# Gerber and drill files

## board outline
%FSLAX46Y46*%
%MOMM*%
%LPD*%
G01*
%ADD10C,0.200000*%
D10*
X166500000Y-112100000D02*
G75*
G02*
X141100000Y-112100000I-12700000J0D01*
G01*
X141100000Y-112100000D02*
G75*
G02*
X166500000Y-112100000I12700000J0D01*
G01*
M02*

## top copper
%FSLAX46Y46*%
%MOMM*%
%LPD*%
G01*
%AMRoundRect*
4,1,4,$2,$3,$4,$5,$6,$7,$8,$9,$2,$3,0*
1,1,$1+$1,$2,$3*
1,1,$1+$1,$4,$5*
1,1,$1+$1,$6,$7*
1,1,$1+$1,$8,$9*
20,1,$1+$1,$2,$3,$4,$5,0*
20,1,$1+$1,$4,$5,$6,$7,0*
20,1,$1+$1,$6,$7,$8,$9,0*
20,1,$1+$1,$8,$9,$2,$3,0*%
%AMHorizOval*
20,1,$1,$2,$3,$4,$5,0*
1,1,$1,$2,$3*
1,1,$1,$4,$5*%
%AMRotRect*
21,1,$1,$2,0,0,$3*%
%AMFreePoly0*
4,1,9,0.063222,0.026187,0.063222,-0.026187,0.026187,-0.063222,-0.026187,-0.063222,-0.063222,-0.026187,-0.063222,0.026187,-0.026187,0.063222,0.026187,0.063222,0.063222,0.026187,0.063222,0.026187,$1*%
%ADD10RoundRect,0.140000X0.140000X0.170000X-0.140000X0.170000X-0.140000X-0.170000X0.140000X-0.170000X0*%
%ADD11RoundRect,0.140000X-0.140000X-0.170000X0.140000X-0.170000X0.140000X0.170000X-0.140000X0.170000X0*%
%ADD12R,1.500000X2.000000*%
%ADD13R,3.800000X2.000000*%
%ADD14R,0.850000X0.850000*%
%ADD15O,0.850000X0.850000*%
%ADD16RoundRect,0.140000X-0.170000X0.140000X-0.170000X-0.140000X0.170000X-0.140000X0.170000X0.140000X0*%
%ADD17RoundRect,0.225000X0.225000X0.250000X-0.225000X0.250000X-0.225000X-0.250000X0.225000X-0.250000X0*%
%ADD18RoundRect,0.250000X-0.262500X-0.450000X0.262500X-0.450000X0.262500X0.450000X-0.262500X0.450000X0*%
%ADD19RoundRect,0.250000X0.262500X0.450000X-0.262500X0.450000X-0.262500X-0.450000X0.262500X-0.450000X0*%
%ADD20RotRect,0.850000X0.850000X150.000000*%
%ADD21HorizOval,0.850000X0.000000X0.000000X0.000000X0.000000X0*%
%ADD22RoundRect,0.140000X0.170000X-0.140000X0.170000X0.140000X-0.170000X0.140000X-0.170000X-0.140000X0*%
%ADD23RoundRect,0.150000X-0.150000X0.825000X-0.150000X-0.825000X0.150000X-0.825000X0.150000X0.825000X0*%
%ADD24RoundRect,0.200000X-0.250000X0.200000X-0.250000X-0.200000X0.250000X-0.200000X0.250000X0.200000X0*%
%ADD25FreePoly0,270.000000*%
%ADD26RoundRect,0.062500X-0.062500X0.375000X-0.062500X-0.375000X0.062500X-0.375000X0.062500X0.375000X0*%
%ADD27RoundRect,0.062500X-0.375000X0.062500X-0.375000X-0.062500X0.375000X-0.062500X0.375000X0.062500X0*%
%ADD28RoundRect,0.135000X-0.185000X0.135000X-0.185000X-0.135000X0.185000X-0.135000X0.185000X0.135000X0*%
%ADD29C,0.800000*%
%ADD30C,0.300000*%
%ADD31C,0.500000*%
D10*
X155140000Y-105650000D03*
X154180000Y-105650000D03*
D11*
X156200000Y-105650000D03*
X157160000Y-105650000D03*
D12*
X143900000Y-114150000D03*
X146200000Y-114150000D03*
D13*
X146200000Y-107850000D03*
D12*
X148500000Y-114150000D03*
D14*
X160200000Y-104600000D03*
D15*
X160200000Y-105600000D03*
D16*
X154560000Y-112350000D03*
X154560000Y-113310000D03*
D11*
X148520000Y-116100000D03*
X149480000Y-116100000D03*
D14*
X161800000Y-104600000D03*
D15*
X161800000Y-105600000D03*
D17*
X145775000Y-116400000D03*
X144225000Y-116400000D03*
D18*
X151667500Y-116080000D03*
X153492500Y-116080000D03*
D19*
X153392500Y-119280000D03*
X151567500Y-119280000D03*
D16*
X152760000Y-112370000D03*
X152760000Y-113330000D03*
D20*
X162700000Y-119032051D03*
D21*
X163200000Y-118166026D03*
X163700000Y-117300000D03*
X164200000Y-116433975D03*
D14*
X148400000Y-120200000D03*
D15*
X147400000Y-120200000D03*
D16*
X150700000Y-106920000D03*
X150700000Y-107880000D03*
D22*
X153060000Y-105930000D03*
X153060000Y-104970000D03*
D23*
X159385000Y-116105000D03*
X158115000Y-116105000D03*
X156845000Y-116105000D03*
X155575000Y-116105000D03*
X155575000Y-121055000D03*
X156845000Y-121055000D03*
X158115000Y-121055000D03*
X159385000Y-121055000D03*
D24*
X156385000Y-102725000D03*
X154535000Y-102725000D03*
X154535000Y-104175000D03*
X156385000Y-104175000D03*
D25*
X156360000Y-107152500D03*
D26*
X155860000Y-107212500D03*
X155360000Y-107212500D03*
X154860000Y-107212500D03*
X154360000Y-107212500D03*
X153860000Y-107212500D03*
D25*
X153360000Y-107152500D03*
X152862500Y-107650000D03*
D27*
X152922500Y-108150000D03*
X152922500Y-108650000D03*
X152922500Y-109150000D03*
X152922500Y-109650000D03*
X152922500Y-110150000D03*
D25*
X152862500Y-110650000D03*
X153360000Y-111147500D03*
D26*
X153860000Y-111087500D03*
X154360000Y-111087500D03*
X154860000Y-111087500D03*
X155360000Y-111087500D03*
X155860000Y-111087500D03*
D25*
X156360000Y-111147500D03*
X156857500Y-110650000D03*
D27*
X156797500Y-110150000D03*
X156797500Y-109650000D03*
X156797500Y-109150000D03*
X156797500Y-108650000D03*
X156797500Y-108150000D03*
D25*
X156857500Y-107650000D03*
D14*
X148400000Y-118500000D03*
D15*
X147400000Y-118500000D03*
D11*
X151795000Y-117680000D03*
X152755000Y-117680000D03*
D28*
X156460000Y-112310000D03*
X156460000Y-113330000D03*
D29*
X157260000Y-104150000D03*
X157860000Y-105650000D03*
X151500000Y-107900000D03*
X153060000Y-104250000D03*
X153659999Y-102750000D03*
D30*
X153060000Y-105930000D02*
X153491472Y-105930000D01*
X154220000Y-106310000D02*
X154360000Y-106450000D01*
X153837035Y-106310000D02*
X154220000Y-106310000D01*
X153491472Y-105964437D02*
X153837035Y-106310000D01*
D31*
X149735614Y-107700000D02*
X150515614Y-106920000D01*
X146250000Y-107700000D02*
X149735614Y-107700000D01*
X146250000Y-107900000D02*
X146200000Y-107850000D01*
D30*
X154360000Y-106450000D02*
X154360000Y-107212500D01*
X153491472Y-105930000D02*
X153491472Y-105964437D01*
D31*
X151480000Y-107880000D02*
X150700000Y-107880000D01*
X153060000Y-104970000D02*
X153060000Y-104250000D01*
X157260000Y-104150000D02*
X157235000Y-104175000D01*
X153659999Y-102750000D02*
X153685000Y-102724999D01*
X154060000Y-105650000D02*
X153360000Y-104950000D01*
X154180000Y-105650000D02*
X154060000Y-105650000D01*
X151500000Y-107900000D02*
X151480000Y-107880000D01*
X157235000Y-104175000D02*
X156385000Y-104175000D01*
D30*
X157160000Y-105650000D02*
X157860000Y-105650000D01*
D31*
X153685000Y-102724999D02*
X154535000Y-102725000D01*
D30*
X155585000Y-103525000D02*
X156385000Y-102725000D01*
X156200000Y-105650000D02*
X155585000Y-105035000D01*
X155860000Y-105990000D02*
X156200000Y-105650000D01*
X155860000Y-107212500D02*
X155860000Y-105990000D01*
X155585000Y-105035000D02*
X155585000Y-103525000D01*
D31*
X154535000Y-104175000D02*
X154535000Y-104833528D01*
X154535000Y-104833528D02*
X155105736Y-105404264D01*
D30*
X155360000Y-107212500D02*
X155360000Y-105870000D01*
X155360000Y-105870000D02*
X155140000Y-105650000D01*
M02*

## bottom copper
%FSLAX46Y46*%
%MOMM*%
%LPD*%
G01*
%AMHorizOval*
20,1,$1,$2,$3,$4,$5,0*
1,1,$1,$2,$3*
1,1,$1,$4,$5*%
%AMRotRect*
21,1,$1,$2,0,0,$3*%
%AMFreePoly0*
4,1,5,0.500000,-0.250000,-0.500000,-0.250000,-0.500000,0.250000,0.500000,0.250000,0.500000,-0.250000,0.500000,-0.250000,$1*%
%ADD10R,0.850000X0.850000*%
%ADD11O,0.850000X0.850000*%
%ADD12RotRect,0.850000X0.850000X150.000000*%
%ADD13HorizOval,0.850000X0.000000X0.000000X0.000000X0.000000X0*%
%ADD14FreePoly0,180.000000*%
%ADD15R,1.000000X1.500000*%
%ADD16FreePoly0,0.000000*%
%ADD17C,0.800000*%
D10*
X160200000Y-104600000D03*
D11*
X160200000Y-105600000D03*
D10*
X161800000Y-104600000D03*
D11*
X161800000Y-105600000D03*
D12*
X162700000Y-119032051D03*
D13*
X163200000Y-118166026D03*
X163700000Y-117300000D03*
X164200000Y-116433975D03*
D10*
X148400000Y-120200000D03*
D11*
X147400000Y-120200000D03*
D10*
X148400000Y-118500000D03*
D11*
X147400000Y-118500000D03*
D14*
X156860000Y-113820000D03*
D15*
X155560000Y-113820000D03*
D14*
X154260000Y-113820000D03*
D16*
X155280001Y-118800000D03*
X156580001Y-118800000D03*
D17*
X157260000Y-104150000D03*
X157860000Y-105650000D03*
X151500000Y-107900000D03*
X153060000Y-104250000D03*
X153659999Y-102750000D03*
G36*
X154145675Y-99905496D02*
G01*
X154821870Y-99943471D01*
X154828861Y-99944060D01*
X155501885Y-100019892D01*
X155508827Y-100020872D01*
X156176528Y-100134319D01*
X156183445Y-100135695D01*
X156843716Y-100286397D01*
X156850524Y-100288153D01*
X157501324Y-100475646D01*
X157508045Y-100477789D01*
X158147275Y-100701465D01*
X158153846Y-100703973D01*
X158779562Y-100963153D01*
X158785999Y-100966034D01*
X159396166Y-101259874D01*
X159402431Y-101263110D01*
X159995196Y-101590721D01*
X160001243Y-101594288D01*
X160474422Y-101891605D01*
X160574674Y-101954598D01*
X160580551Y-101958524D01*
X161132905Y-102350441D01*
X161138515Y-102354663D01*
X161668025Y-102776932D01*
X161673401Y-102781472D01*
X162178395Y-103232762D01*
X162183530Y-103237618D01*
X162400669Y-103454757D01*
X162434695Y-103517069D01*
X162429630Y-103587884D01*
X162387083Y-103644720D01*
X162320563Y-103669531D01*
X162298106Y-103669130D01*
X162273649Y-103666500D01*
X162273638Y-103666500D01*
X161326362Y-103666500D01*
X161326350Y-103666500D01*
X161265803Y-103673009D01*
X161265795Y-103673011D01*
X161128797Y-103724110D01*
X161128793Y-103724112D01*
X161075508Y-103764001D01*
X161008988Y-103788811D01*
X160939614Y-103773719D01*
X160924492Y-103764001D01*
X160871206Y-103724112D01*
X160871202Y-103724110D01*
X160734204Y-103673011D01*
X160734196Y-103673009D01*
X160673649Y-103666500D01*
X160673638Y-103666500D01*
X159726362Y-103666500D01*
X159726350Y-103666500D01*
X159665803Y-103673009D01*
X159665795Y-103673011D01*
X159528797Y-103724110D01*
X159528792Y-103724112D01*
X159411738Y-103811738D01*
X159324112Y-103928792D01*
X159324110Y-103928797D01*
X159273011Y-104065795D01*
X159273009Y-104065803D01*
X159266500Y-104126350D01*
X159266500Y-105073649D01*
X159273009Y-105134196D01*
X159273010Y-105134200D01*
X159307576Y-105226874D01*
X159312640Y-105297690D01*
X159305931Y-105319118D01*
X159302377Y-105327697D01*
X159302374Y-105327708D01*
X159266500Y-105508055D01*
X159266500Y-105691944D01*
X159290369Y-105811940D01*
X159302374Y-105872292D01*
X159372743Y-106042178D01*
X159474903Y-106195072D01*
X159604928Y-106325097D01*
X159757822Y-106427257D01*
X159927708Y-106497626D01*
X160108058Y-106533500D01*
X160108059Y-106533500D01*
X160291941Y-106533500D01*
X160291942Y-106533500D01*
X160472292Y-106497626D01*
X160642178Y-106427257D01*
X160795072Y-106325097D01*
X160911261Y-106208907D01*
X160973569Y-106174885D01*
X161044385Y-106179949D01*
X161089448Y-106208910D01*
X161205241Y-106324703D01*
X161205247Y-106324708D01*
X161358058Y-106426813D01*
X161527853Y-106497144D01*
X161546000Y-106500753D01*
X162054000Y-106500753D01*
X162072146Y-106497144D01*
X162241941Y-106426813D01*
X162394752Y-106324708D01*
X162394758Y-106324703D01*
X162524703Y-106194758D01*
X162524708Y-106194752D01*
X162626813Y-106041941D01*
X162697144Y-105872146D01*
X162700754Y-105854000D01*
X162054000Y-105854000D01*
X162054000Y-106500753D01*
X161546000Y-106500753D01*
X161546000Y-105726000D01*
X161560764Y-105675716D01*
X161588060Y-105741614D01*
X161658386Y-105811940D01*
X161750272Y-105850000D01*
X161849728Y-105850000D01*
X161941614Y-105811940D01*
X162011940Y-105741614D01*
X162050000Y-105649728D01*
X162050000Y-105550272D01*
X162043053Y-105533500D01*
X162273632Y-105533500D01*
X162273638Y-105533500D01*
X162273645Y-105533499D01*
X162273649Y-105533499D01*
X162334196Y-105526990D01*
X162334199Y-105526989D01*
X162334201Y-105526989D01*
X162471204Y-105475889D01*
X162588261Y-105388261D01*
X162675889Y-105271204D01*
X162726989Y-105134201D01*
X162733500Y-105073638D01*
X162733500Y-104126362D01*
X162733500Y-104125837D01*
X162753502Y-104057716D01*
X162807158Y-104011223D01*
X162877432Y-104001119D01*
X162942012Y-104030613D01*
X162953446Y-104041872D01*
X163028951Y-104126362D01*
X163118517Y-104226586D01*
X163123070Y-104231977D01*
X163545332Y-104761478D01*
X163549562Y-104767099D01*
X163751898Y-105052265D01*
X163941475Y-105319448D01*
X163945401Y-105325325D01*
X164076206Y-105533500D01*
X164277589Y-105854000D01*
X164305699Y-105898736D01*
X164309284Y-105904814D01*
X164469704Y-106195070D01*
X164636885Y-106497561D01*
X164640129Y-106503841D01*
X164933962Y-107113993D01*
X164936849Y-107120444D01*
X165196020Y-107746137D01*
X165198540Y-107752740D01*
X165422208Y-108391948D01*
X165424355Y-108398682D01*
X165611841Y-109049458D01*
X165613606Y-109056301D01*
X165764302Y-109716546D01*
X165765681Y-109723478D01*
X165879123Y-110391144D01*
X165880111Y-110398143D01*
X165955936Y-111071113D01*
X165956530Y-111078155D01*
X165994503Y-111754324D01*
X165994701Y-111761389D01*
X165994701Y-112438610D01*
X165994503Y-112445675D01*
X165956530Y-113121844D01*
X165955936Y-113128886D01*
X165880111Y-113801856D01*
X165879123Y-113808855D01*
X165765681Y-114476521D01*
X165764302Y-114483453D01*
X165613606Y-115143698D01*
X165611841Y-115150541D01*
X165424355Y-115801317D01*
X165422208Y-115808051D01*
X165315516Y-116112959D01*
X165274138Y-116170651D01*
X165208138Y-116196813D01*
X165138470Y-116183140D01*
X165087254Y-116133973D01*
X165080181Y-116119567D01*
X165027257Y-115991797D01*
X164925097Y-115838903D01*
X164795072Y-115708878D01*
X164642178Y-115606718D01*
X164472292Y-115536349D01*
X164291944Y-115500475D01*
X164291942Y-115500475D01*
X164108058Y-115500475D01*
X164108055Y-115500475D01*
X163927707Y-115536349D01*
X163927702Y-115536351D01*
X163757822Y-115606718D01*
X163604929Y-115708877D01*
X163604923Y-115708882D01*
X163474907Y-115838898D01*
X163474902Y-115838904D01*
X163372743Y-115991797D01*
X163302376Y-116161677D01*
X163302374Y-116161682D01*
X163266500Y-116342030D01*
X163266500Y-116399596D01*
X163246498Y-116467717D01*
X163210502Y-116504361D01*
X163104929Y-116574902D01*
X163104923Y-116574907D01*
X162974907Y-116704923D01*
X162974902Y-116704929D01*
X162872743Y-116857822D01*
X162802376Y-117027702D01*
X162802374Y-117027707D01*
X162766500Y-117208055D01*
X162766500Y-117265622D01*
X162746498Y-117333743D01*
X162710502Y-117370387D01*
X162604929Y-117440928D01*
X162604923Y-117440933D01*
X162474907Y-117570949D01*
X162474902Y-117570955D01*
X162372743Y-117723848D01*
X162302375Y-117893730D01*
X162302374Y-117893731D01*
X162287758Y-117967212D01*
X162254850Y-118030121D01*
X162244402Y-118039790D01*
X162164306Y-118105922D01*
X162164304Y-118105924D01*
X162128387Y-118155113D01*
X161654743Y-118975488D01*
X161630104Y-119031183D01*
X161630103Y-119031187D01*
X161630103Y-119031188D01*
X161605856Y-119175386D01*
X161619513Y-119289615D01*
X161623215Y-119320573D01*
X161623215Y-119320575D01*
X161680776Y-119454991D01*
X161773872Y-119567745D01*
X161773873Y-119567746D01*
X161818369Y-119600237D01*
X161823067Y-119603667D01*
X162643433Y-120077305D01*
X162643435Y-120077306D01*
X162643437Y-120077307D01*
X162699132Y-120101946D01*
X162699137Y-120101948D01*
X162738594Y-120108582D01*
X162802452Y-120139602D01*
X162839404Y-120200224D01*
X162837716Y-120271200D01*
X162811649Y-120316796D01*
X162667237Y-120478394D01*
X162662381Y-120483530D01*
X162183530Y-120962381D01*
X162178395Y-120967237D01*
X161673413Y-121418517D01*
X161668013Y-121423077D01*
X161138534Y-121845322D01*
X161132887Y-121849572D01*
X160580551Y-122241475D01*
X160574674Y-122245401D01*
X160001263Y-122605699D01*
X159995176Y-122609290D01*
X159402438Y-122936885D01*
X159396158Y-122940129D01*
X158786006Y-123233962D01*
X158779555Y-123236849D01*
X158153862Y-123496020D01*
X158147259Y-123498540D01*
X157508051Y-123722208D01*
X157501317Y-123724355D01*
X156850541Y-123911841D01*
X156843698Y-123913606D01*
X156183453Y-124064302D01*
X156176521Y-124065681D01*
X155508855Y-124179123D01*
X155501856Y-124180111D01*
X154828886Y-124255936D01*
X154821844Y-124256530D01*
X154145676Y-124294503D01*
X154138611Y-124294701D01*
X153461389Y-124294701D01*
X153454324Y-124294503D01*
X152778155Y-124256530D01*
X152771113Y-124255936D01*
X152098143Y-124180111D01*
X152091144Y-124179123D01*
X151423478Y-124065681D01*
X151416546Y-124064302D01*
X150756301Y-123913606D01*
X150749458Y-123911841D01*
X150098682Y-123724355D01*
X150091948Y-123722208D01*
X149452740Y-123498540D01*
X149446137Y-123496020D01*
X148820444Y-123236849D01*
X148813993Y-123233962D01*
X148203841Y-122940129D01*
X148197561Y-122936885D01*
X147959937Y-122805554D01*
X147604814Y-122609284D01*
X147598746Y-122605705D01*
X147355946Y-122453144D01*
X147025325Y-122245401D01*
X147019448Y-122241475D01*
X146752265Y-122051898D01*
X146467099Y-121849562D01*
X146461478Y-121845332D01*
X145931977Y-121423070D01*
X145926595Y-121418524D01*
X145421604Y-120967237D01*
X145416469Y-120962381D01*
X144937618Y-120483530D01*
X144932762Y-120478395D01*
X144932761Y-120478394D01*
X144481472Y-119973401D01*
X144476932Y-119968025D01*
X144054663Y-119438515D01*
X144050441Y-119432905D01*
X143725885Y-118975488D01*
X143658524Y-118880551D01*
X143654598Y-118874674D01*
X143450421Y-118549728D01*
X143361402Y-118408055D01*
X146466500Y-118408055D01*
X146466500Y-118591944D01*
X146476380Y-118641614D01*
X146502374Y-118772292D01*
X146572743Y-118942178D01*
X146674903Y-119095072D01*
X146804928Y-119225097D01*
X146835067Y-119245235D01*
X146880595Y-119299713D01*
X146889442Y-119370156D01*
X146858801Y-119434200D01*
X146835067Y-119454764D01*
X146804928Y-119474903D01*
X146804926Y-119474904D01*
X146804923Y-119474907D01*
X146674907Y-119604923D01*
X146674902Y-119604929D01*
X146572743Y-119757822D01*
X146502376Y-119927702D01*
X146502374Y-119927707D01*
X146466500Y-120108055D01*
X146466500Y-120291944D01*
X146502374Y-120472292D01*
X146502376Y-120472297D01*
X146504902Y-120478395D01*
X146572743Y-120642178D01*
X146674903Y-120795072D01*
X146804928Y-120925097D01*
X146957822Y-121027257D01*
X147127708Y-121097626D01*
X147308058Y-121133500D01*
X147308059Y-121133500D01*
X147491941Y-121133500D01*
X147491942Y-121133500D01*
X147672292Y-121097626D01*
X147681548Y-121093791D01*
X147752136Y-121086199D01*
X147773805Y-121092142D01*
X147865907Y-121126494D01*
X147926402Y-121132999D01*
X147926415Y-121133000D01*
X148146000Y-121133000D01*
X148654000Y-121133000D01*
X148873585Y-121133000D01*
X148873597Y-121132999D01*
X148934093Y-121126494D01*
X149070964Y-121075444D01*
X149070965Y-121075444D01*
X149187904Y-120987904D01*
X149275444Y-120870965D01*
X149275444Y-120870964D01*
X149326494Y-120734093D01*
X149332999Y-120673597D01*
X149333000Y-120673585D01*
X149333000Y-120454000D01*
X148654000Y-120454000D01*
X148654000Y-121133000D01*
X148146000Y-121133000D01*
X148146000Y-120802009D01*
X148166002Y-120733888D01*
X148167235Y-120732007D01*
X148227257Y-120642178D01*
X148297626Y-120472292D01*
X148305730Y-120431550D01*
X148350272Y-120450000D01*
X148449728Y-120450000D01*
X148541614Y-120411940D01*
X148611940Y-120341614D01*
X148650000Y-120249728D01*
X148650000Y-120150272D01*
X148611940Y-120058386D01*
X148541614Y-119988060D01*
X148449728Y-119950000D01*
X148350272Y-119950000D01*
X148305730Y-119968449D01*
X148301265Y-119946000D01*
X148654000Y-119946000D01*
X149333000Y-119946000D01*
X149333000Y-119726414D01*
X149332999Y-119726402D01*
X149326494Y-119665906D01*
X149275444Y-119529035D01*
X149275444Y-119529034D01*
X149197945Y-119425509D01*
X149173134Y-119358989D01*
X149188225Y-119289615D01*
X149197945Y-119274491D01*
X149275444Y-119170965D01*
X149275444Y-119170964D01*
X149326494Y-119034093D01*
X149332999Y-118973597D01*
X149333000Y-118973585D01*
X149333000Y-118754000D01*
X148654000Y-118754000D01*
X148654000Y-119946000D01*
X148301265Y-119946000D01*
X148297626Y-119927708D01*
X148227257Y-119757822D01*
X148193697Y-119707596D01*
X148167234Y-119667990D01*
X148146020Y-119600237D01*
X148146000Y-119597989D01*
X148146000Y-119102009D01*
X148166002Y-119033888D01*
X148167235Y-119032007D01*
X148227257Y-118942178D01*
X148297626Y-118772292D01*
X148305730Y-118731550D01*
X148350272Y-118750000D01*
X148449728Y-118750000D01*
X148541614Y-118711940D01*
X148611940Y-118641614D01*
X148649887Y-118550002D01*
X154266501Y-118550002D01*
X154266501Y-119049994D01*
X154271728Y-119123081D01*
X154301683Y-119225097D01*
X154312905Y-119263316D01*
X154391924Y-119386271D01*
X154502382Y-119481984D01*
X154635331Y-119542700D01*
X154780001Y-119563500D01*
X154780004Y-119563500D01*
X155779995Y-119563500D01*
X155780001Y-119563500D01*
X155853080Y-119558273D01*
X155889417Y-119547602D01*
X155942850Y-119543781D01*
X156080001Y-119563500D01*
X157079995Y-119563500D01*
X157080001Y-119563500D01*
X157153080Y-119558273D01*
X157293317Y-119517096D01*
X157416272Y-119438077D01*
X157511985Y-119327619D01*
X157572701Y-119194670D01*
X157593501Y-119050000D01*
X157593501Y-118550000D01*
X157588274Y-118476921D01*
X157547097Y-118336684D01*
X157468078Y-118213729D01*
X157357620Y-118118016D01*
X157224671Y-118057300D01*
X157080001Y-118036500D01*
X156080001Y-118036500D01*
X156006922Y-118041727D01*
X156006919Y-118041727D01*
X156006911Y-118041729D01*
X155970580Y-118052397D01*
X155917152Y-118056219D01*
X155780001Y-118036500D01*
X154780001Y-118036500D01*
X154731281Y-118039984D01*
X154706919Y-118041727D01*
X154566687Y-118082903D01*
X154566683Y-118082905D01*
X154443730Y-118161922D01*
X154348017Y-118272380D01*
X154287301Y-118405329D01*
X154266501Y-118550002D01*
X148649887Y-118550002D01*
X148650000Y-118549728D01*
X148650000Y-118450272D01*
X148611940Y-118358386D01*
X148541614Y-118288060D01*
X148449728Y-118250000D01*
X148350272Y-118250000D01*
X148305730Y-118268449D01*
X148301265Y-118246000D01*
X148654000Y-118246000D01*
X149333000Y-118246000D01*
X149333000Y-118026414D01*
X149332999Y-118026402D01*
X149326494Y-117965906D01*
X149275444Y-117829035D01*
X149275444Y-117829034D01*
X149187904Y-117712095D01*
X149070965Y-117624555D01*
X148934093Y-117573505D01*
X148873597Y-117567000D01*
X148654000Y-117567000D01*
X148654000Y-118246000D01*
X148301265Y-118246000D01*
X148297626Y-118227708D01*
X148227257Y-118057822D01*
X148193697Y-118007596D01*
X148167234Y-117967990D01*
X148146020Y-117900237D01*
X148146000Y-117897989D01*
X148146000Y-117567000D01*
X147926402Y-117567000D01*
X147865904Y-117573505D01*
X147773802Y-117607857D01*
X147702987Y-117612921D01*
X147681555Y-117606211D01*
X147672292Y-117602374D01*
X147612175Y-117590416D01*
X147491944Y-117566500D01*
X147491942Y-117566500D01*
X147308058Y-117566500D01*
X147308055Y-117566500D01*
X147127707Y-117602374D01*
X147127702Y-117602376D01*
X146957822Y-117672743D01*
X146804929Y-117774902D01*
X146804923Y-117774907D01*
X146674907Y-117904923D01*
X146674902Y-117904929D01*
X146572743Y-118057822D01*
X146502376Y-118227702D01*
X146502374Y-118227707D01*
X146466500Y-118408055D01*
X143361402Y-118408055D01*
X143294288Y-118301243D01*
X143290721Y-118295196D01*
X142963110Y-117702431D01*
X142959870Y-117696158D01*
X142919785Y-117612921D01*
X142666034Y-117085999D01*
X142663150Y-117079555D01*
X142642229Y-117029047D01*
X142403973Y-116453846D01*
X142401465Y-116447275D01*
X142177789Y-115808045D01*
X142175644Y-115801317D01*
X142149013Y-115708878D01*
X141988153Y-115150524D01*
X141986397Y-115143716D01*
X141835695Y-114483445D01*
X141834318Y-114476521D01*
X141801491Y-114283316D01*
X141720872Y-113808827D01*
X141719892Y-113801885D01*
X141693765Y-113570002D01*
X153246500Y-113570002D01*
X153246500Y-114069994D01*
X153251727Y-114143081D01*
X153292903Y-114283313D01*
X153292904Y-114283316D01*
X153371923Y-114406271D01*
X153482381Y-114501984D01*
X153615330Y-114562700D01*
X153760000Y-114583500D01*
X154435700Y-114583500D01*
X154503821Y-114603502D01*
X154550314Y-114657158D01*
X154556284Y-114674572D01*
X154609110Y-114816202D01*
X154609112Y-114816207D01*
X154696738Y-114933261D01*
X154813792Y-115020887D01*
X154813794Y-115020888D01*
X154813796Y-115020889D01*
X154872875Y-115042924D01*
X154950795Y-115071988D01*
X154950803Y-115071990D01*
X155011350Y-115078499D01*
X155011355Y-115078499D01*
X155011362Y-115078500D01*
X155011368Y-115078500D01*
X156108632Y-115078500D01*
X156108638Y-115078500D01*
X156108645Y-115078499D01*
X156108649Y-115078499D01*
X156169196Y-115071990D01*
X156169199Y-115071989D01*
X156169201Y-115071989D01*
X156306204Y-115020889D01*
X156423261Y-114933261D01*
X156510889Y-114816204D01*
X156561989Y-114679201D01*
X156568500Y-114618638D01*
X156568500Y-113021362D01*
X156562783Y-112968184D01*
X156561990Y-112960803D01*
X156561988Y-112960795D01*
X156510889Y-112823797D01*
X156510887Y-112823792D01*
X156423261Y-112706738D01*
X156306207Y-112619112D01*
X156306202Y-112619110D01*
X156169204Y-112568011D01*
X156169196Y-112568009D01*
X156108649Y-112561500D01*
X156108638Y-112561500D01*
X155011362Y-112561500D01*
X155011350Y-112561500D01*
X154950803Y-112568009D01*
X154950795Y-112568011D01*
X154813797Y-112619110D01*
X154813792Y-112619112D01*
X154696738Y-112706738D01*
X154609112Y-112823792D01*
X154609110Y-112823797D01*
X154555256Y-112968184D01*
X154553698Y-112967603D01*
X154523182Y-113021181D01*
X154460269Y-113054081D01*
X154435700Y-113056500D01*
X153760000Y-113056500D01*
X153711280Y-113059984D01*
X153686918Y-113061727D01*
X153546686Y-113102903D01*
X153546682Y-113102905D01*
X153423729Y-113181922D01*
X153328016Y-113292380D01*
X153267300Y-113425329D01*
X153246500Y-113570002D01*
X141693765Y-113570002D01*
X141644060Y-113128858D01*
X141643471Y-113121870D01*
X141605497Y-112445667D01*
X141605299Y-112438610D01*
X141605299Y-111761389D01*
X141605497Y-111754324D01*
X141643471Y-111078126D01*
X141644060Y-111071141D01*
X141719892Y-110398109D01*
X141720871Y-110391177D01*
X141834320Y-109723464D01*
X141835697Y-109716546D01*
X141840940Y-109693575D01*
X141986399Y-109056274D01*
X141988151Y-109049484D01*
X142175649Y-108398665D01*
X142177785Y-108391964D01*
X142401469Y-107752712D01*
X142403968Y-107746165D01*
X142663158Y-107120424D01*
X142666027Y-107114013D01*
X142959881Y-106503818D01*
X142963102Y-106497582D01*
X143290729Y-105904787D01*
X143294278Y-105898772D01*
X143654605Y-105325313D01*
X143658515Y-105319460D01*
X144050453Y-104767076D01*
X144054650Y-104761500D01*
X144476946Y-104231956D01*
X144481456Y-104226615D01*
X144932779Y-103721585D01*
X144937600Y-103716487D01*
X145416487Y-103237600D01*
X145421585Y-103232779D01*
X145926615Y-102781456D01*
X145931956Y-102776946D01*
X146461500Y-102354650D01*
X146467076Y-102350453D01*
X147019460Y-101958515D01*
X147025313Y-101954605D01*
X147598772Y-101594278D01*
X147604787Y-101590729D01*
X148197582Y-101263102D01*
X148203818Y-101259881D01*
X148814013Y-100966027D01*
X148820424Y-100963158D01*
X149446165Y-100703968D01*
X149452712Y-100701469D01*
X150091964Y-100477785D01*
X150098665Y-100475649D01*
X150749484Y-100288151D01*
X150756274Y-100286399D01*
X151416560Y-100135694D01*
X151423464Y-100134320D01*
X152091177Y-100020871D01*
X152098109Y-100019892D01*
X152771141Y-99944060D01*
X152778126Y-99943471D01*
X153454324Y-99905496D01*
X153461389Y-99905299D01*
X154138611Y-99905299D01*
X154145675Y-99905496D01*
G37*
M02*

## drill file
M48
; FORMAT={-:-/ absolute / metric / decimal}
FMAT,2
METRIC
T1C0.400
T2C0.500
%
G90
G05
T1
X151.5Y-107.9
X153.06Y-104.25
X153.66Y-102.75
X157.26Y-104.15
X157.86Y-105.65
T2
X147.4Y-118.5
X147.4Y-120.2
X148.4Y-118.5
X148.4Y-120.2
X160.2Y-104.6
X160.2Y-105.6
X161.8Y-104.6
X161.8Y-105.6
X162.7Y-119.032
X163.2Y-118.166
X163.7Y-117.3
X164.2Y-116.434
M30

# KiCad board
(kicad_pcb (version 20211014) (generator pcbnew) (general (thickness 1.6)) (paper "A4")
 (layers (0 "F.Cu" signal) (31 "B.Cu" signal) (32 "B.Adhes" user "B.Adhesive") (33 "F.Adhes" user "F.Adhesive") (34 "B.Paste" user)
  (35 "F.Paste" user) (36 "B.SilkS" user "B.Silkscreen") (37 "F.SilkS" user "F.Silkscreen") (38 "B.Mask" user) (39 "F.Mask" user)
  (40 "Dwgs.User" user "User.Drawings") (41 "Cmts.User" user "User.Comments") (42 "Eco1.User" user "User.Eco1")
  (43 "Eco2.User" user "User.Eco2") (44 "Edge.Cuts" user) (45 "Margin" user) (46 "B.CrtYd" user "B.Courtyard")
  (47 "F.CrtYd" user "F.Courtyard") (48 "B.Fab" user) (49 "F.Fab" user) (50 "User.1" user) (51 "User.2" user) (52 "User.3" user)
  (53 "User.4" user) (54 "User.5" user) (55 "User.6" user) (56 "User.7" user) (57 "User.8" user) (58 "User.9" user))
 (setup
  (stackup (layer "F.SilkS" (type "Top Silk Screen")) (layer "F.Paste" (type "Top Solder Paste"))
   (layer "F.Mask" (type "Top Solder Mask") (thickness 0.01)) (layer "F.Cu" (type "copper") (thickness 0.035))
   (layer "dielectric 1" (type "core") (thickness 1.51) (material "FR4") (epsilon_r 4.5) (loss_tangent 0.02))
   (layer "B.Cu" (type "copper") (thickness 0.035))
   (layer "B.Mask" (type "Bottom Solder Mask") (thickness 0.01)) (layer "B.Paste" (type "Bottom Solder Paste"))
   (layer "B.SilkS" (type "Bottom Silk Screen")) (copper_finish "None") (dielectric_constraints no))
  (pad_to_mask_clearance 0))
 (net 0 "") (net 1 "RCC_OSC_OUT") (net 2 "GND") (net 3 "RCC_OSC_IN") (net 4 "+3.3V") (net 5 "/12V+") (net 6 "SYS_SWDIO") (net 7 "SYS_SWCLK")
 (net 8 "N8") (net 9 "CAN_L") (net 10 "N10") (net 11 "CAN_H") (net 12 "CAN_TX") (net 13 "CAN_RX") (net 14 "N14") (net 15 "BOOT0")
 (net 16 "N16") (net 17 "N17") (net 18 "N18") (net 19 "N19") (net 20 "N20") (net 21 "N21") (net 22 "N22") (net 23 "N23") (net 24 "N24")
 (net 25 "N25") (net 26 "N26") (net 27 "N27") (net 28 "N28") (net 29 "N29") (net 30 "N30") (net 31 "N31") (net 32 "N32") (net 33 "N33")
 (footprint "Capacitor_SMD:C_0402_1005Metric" (layer "F.Cu") (at 154.66 105.65 180)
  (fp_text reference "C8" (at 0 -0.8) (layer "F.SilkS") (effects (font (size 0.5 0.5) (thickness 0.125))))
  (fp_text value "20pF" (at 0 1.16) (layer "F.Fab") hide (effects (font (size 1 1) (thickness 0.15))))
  (pad "1" smd roundrect (at -0.48 0 180) (size 0.56 0.62) (layers "F.Cu" "F.Paste" "F.Mask") (roundrect_rratio 0.25) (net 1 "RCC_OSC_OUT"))
  (pad "2" smd roundrect (at 0.48 0 180) (size 0.56 0.62) (layers "F.Cu" "F.Paste" "F.Mask") (roundrect_rratio 0.25) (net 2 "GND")))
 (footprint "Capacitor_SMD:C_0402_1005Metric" (layer "F.Cu") (at 156.68 105.65)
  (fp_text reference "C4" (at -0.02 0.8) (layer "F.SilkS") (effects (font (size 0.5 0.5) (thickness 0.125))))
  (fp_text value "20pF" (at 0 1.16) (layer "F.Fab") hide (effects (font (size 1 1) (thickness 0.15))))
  (pad "1" smd roundrect (at -0.48 0) (size 0.56 0.62) (layers "F.Cu" "F.Paste" "F.Mask") (roundrect_rratio 0.25) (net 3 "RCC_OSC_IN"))
  (pad "2" smd roundrect (at 0.48 0) (size 0.56 0.62) (layers "F.Cu" "F.Paste" "F.Mask") (roundrect_rratio 0.25) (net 2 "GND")))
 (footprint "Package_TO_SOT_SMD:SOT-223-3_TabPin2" (layer "F.Cu") (at 146.2 111 90)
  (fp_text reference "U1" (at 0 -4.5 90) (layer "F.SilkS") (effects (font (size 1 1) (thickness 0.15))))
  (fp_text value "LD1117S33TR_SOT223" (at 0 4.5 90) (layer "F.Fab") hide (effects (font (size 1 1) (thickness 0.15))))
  (pad "1" smd rect (at -3.15 -2.3 90) (size 2 1.5) (layers "F.Cu" "F.Paste" "F.Mask") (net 2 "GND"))
  (pad "2" smd rect (at -3.15 0 90) (size 2 1.5) (layers "F.Cu" "F.Paste" "F.Mask") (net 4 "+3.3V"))
  (pad "2" smd rect (at 3.15 0 90) (size 2 3.8) (layers "F.Cu" "F.Paste" "F.Mask") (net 4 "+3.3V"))
  (pad "3" smd rect (at -3.15 2.3 90) (size 2 1.5) (layers "F.Cu" "F.Paste" "F.Mask") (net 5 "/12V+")))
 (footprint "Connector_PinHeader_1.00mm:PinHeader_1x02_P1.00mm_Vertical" (layer "F.Cu") (at 160.2 104.6)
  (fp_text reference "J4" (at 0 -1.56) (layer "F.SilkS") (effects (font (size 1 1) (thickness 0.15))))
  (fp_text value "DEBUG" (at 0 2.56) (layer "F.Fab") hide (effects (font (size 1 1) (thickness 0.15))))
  (pad "1" thru_hole rect (at 0 0) (size 0.85 0.85) (drill 0.5) (layers *.Cu *.Mask) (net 4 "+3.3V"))
  (pad "2" thru_hole oval (at 0 1) (size 0.85 0.85) (drill 0.5) (layers *.Cu *.Mask) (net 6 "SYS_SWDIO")))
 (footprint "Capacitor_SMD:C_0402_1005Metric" (layer "F.Cu") (at 154.56 112.83 -90)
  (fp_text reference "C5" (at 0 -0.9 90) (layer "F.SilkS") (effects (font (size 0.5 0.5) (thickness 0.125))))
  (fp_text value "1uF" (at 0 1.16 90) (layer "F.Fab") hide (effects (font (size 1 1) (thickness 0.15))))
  (pad "1" smd roundrect (at -0.48 0 270) (size 0.56 0.62) (layers "F.Cu" "F.Paste" "F.Mask") (roundrect_rratio 0.25) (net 4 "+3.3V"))
  (pad "2" smd roundrect (at 0.48 0 270) (size 0.56 0.62) (layers "F.Cu" "F.Paste" "F.Mask") (roundrect_rratio 0.25) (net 2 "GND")))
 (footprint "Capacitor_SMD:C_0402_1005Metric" (layer "F.Cu") (at 149 116.1)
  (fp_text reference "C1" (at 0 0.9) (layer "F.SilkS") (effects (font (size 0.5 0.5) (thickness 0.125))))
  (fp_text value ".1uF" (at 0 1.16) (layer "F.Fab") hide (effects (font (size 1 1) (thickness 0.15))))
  (pad "1" smd roundrect (at -0.48 0) (size 0.56 0.62) (layers "F.Cu" "F.Paste" "F.Mask") (roundrect_rratio 0.25) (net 5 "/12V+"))
  (pad "2" smd roundrect (at 0.48 0) (size 0.56 0.62) (layers "F.Cu" "F.Paste" "F.Mask") (roundrect_rratio 0.25) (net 2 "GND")))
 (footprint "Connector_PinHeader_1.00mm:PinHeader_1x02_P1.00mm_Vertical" (layer "F.Cu") (at 161.8 104.6)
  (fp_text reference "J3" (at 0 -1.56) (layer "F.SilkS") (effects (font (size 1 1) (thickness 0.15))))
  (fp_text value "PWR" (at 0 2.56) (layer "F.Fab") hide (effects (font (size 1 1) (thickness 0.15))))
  (pad "1" thru_hole rect (at 0 0) (size 0.85 0.85) (drill 0.5) (layers *.Cu *.Mask) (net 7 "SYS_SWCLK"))
  (pad "2" thru_hole oval (at 0 1) (size 0.85 0.85) (drill 0.5) (layers *.Cu *.Mask) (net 2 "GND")))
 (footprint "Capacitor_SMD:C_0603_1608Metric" (layer "F.Cu") (at 145 116.4 180)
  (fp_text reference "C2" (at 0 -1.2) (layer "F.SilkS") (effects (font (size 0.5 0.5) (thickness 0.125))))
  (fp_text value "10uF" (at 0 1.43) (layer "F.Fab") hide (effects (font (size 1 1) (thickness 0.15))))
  (pad "1" smd roundrect (at -0.775 0 180) (size 0.9 0.95) (layers "F.Cu" "F.Paste" "F.Mask") (roundrect_rratio 0.25) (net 4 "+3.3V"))
  (pad "2" smd roundrect (at 0.775 0 180) (size 0.9 0.95) (layers "F.Cu" "F.Paste" "F.Mask") (roundrect_rratio 0.25) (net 2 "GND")))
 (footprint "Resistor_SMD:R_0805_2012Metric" (layer "F.Cu") (at 152.58 116.08)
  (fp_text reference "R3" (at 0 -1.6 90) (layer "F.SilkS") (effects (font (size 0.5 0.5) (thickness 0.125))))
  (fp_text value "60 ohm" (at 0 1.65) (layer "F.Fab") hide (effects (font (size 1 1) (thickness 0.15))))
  (pad "1" smd roundrect (at -0.9125 0) (size 1.025 1.4) (layers "F.Cu" "F.Paste" "F.Mask") (roundrect_rratio 0.243902) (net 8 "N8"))
  (pad "2" smd roundrect (at 0.9125 0) (size 1.025 1.4) (layers "F.Cu" "F.Paste" "F.Mask") (roundrect_rratio 0.243902) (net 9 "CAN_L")))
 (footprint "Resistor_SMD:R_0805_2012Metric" (layer "F.Cu") (at 152.48 119.28 180)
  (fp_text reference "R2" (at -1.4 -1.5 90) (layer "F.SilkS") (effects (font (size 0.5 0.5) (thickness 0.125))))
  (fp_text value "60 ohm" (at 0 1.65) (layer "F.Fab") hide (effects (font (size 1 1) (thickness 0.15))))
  (pad "1" smd roundrect (at -0.9125 0 180) (size 1.025 1.4) (layers "F.Cu" "F.Paste" "F.Mask") (roundrect_rratio 0.243902) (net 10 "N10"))
  (pad "2" smd roundrect (at 0.9125 0 180) (size 1.025 1.4) (layers "F.Cu" "F.Paste" "F.Mask") (roundrect_rratio 0.243902) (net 8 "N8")))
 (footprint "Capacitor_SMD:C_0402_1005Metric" (layer "F.Cu") (at 152.76 112.85 -90)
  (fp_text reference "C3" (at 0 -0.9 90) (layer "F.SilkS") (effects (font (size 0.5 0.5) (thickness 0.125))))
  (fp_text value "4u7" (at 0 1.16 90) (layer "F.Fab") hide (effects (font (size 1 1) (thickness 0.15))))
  (pad "1" smd roundrect (at -0.48 0 270) (size 0.56 0.62) (layers "F.Cu" "F.Paste" "F.Mask") (roundrect_rratio 0.25) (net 4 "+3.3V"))
  (pad "2" smd roundrect (at 0.48 0 270) (size 0.56 0.62) (layers "F.Cu" "F.Paste" "F.Mask") (roundrect_rratio 0.25) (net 2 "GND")))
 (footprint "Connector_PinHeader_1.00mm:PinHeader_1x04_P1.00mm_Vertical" (layer "F.Cu") (at 162.7 119.032051 150)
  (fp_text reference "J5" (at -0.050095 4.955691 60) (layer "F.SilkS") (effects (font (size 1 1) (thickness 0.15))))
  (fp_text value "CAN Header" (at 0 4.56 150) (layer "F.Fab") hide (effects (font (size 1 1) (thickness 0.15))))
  (pad "1" thru_hole rect (at 0 0 150) (size 0.85 0.85) (drill 0.5) (layers *.Cu *.Mask) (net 9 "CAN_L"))
  (pad "2" thru_hole oval (at 0 1 150) (size 0.85 0.85) (drill 0.5) (layers *.Cu *.Mask) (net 9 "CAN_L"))
  (pad "3" thru_hole oval (at 0 2 150) (size 0.85 0.85) (drill 0.5) (layers *.Cu *.Mask) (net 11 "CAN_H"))
  (pad "4" thru_hole oval (at 0 3 150) (size 0.85 0.85) (drill 0.5) (layers *.Cu *.Mask) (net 11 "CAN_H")))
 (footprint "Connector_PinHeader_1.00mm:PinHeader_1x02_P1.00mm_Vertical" (layer "F.Cu") (at 148.4 120.2 -90)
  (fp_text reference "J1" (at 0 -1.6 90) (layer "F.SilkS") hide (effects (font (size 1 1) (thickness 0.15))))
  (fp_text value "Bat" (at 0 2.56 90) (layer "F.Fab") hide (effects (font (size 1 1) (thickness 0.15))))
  (pad "1" thru_hole rect (at 0 0 270) (size 0.85 0.85) (drill 0.5) (layers *.Cu *.Mask) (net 2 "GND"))
  (pad "2" thru_hole oval (at 0 1 270) (size 0.85 0.85) (drill 0.5) (layers *.Cu *.Mask) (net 5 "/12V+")))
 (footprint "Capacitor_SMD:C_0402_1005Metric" (layer "F.Cu") (at 150.7 107.4 -90)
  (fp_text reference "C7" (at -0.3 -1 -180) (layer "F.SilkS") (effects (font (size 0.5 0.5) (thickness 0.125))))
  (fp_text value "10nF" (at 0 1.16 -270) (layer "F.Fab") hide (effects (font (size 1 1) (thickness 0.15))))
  (pad "1" smd roundrect (at -0.48 0 270) (size 0.56 0.62) (layers "F.Cu" "F.Paste" "F.Mask") (roundrect_rratio 0.25) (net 4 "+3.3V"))
  (pad "2" smd roundrect (at 0.48 0 270) (size 0.56 0.62) (layers "F.Cu" "F.Paste" "F.Mask") (roundrect_rratio 0.25) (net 2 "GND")))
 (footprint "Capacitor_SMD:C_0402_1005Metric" (layer "F.Cu") (at 153.06 105.45 90)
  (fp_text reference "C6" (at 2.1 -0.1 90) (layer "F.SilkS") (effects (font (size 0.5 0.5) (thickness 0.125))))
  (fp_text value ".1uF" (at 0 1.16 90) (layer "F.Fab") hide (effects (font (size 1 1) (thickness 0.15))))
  (pad "1" smd roundrect (at -0.48 0 90) (size 0.56 0.62) (layers "F.Cu" "F.Paste" "F.Mask") (roundrect_rratio 0.25) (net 4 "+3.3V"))
  (pad "2" smd roundrect (at 0.48 0 90) (size 0.56 0.62) (layers "F.Cu" "F.Paste" "F.Mask") (roundrect_rratio 0.25) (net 2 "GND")))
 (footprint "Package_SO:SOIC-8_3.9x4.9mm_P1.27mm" (layer "F.Cu") (at 157.48 118.58 -90)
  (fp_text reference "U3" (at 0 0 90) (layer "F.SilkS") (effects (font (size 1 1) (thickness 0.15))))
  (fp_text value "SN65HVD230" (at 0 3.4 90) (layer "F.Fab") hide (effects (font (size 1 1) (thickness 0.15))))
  (pad "1" smd roundrect (at -2.475 -1.905 270) (size 1.95 0.6) (layers "F.Cu" "F.Paste" "F.Mask") (roundrect_rratio 0.25) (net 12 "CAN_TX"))
  (pad "2" smd roundrect (at -2.475 -0.635 270) (size 1.95 0.6) (layers "F.Cu" "F.Paste" "F.Mask") (roundrect_rratio 0.25) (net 2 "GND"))
  (pad "3" smd roundrect (at -2.475 0.635 270) (size 1.95 0.6) (layers "F.Cu" "F.Paste" "F.Mask") (roundrect_rratio 0.25) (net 4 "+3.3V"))
  (pad "4" smd roundrect (at -2.475 1.905 270) (size 1.95 0.6) (layers "F.Cu" "F.Paste" "F.Mask") (roundrect_rratio 0.25) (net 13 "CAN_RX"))
  (pad "5" smd roundrect (at 2.475 1.905 270) (size 1.95 0.6) (layers "F.Cu" "F.Paste" "F.Mask") (roundrect_rratio 0.25) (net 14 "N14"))
  (pad "6" smd roundrect (at 2.475 0.635 270) (size 1.95 0.6) (layers "F.Cu" "F.Paste" "F.Mask") (roundrect_rratio 0.25) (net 9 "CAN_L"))
  (pad "7" smd roundrect (at 2.475 -0.635 270) (size 1.95 0.6) (layers "F.Cu" "F.Paste" "F.Mask") (roundrect_rratio 0.25) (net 11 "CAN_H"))
  (pad "8" smd roundrect (at 2.475 -1.905 270) (size 1.95 0.6) (layers "F.Cu" "F.Paste" "F.Mask") (roundrect_rratio 0.25) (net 2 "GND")))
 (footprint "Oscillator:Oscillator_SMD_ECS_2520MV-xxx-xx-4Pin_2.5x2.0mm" (layer "F.Cu") (at 155.46 103.45 -90)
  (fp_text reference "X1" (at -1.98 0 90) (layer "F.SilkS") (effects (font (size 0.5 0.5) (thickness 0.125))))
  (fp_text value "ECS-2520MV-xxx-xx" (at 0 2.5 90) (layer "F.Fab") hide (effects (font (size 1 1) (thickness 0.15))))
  (pad "1" smd roundrect (at -0.725 -0.925 270) (size 0.8 0.9) (layers "F.Cu" "F.Paste" "F.Mask") (roundrect_rratio 0.25)
   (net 3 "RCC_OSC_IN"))
  (pad "2" smd roundrect (at -0.725 0.925 270) (size 0.8 0.9) (layers "F.Cu" "F.Paste" "F.Mask") (roundrect_rratio 0.25) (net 2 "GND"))
  (pad "3" smd roundrect (at 0.725 0.925 270) (size 0.8 0.9) (layers "F.Cu" "F.Paste" "F.Mask") (roundrect_rratio 0.25)
   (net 1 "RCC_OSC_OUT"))
  (pad "4" smd roundrect (at 0.725 -0.925 270) (size 0.8 0.9) (layers "F.Cu" "F.Paste" "F.Mask") (roundrect_rratio 0.25) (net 2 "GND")))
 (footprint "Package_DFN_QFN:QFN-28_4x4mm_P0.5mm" (layer "F.Cu") (at 154.86 109.15 -90)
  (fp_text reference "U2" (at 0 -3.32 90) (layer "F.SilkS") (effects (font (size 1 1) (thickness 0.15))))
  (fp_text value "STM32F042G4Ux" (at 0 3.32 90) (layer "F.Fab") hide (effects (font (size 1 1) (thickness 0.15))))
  (pad "1" smd custom (at -1.9975 -1.5 270) (size 0.136863 0.136863) (layers "F.Cu" "F.Paste" "F.Mask") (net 13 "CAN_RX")
   (options (clearance outline) (anchor circle)) (primitives))
  (pad "2" smd roundrect (at -1.9375 -1 270) (size 0.875 0.25) (layers "F.Cu" "F.Paste" "F.Mask") (roundrect_rratio 0.25)
   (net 3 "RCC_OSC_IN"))
  (pad "3" smd roundrect (at -1.9375 -0.5 270) (size 0.875 0.25) (layers "F.Cu" "F.Paste" "F.Mask") (roundrect_rratio 0.25)
   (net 1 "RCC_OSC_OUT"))
  (pad "4" smd roundrect (at -1.9375 0 270) (size 0.875 0.25) (layers "F.Cu" "F.Paste" "F.Mask") (roundrect_rratio 0.25) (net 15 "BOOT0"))
  (pad "5" smd roundrect (at -1.9375 0.5 270) (size 0.875 0.25) (layers "F.Cu" "F.Paste" "F.Mask") (roundrect_rratio 0.25) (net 4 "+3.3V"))
  (pad "6" smd roundrect (at -1.9375 1 270) (size 0.875 0.25) (layers "F.Cu" "F.Paste" "F.Mask") (roundrect_rratio 0.25) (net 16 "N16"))
  (pad "7" smd custom (at -1.9975 1.5 270) (size 0.136863 0.136863) (layers "F.Cu" "F.Paste" "F.Mask") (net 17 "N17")
   (options (clearance outline) (anchor circle)) (primitives))
  (pad "8" smd custom (at -1.5 1.9975 270) (size 0.136863 0.136863) (layers "F.Cu" "F.Paste" "F.Mask") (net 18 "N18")
   (options (clearance outline) (anchor circle)) (primitives))
  (pad "9" smd roundrect (at -1 1.9375 270) (size 0.25 0.875) (layers "F.Cu" "F.Paste" "F.Mask") (roundrect_rratio 0.25) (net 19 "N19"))
  (pad "10" smd roundrect (at -0.5 1.9375 270) (size 0.25 0.875) (layers "F.Cu" "F.Paste" "F.Mask") (roundrect_rratio 0.25) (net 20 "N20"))
  (pad "11" smd roundrect (at 0 1.9375 270) (size 0.25 0.875) (layers "F.Cu" "F.Paste" "F.Mask") (roundrect_rratio 0.25) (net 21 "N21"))
  (pad "12" smd roundrect (at 0.5 1.9375 270) (size 0.25 0.875) (layers "F.Cu" "F.Paste" "F.Mask") (roundrect_rratio 0.25) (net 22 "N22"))
  (pad "13" smd roundrect (at 1 1.9375 270) (size 0.25 0.875) (layers "F.Cu" "F.Paste" "F.Mask") (roundrect_rratio 0.25) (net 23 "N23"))
  (pad "14" smd custom (at 1.5 1.9975 270) (size 0.136863 0.136863) (layers "F.Cu" "F.Paste" "F.Mask") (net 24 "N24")
   (options (clearance outline) (anchor circle)) (primitives))
  (pad "15" smd custom (at 1.9975 1.5 270) (size 0.136863 0.136863) (layers "F.Cu" "F.Paste" "F.Mask") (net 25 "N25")
   (options (clearance outline) (anchor circle)) (primitives))
  (pad "16" smd roundrect (at 1.9375 1 270) (size 0.875 0.25) (layers "F.Cu" "F.Paste" "F.Mask") (roundrect_rratio 0.25) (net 2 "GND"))
  (pad "17" smd roundrect (at 1.9375 0.5 270) (size 0.875 0.25) (layers "F.Cu" "F.Paste" "F.Mask") (roundrect_rratio 0.25) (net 4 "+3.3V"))
  (pad "18" smd roundrect (at 1.9375 0 270) (size 0.875 0.25) (layers "F.Cu" "F.Paste" "F.Mask") (roundrect_rratio 0.25) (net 4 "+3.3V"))
  (pad "19" smd roundrect (at 1.9375 -0.5 270) (size 0.875 0.25) (layers "F.Cu" "F.Paste" "F.Mask") (roundrect_rratio 0.25) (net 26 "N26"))
  (pad "20" smd roundrect (at 1.9375 -1 270) (size 0.875 0.25) (layers "F.Cu" "F.Paste" "F.Mask") (roundrect_rratio 0.25) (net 12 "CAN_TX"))
  (pad "21" smd custom (at 1.9975 -1.5 270) (size 0.136863 0.136863) (layers "F.Cu" "F.Paste" "F.Mask") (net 6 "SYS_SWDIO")
   (options (clearance outline) (anchor circle)) (primitives))
  (pad "22" smd custom (at 1.5 -1.9975 270) (size 0.136863 0.136863) (layers "F.Cu" "F.Paste" "F.Mask") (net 7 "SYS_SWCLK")
   (options (clearance outline) (anchor circle)) (primitives))
  (pad "23" smd roundrect (at 1 -1.9375 270) (size 0.25 0.875) (layers "F.Cu" "F.Paste" "F.Mask") (roundrect_rratio 0.25) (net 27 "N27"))
  (pad "24" smd roundrect (at 0.5 -1.9375 270) (size 0.25 0.875) (layers "F.Cu" "F.Paste" "F.Mask") (roundrect_rratio 0.25) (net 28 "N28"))
  (pad "25" smd roundrect (at 0 -1.9375 270) (size 0.25 0.875) (layers "F.Cu" "F.Paste" "F.Mask") (roundrect_rratio 0.25) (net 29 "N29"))
  (pad "26" smd roundrect (at -0.5 -1.9375 270) (size 0.25 0.875) (layers "F.Cu" "F.Paste" "F.Mask") (roundrect_rratio 0.25) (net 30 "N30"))
  (pad "27" smd roundrect (at -1 -1.9375 270) (size 0.25 0.875) (layers "F.Cu" "F.Paste" "F.Mask") (roundrect_rratio 0.25) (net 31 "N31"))
  (pad "28" smd custom (at -1.5 -1.9975 270) (size 0.136863 0.136863) (layers "F.Cu" "F.Paste" "F.Mask") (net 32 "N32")
   (options (clearance outline) (anchor circle)) (primitives)))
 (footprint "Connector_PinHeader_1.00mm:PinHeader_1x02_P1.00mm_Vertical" (layer "F.Cu") (at 148.4 118.5 -90)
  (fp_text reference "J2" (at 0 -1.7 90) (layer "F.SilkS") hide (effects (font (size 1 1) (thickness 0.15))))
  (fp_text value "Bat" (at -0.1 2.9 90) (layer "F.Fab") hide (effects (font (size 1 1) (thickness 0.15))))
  (pad "1" thru_hole rect (at 0 0 270) (size 0.85 0.85) (drill 0.5) (layers *.Cu *.Mask) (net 2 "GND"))
  (pad "2" thru_hole oval (at 0 1 270) (size 0.85 0.85) (drill 0.5) (layers *.Cu *.Mask) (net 5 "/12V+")))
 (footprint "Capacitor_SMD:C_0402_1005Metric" (layer "F.Cu") (at 152.275 117.68)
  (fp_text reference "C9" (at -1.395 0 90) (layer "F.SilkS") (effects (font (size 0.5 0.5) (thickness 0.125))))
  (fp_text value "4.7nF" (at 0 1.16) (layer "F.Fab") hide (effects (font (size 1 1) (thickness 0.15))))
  (pad "1" smd roundrect (at -0.48 0) (size 0.56 0.62) (layers "F.Cu" "F.Paste" "F.Mask") (roundrect_rratio 0.25) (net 8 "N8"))
  (pad "2" smd roundrect locked (at 0.48 0) (size 0.56 0.62) (layers "F.Cu" "F.Paste" "F.Mask") (roundrect_rratio 0.25) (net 2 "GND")))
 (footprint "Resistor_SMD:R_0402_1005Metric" (layer "F.Cu") (at 156.46 112.82 -90)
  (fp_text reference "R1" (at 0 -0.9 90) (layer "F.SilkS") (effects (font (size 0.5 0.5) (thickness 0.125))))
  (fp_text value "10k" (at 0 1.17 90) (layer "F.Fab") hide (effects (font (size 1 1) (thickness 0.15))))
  (pad "1" smd roundrect (at -0.51 0 270) (size 0.54 0.64) (layers "F.Cu" "F.Paste" "F.Mask") (roundrect_rratio 0.25) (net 15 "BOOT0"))
  (pad "2" smd roundrect (at 0.51 0 270) (size 0.54 0.64) (layers "F.Cu" "F.Paste" "F.Mask") (roundrect_rratio 0.25) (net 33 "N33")))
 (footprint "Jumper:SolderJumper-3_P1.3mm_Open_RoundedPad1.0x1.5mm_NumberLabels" (layer "B.Cu") (at 155.56 113.82 180)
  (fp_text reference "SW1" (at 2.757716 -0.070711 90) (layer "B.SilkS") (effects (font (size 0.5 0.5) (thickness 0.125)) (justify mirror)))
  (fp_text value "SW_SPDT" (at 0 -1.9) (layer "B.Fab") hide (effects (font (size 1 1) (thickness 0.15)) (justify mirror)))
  (pad "1" smd custom (at -1.3 0 180) (size 1 0.5) (layers "B.Cu" "B.Mask") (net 2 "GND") (zone_connect 2)
   (options (clearance outline) (anchor rect)) (primitives))
  (pad "2" smd rect (at 0 0 180) (size 1 1.5) (layers "B.Cu" "B.Mask") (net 33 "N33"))
  (pad "3" smd custom (at 1.3 0 180) (size 1 0.5) (layers "B.Cu" "B.Mask") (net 4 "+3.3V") (zone_connect 2)
   (options (clearance outline) (anchor rect)) (primitives)))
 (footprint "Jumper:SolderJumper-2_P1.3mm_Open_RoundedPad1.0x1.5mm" (layer "B.Cu") (at 155.930001 118.8)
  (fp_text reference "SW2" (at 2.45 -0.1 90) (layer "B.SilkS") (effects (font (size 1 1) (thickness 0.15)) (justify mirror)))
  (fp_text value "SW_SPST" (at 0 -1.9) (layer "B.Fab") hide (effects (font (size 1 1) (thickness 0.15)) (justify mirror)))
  (pad "1" smd custom (at -0.65 0) (size 1 0.5) (layers "B.Cu" "B.Mask") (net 10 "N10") (zone_connect 2)
   (options (clearance outline) (anchor rect)) (primitives))
  (pad "2" smd custom (at 0.65 0) (size 1 0.5) (layers "B.Cu" "B.Mask") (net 11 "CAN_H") (zone_connect 2)
   (options (clearance outline) (anchor rect)) (primitives)))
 (gr_circle (center 153.8 112.1) (end 166.5 112.1) (layer "Edge.Cuts") (width 0.2) (fill none))
 (segment (start 153.06 105.93) (end 153.491472 105.93) (width 0.3) (layer "F.Cu") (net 4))
 (segment (start 154.22 106.31) (end 154.36 106.45) (width 0.3) (layer "F.Cu") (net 4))
 (segment (start 153.837035 106.31) (end 154.22 106.31) (width 0.3) (layer "F.Cu") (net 4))
 (segment (start 153.491472 105.964437) (end 153.837035 106.31) (width 0.3) (layer "F.Cu") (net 4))
 (segment (start 149.735614 107.7) (end 150.515614 106.92) (width 0.5) (layer "F.Cu") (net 4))
 (segment (start 146.25 107.7) (end 149.735614 107.7) (width 0.5) (layer "F.Cu") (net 4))
 (segment (start 146.25 107.9) (end 146.2 107.85) (width 0.5) (layer "F.Cu") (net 4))
 (segment (start 154.36 106.45) (end 154.36 107.2125) (width 0.3) (layer "F.Cu") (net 4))
 (segment (start 153.491472 105.93) (end 153.491472 105.964437) (width 0.3) (layer "F.Cu") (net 4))
 (segment (start 151.48 107.88) (end 150.7 107.88) (width 0.5) (layer "F.Cu") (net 2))
 (segment (start 153.06 104.97) (end 153.06 104.25) (width 0.5) (layer "F.Cu") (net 2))
 (segment (start 157.26 104.15) (end 157.235 104.175) (width 0.5) (layer "F.Cu") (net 2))
 (segment (start 153.659999 102.75) (end 153.685 102.724999) (width 0.5) (layer "F.Cu") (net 2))
 (segment (start 154.06 105.65) (end 153.36 104.95) (width 0.5) (layer "F.Cu") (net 2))
 (segment (start 154.18 105.65) (end 154.06 105.65) (width 0.5) (layer "F.Cu") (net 2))
 (segment (start 151.5 107.9) (end 151.48 107.88) (width 0.5) (layer "F.Cu") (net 2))
 (segment (start 157.235 104.175) (end 156.385 104.175) (width 0.5) (layer "F.Cu") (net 2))
 (segment (start 157.16 105.65) (end 157.86 105.65) (width 0.3) (layer "F.Cu") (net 2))
 (segment (start 153.685 102.724999) (end 154.535 102.725) (width 0.5) (layer "F.Cu") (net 2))
 (via (at 157.26 104.15) (size 0.8) (drill 0.4) (layers "F.Cu" "B.Cu") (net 2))
 (via (at 157.86 105.65) (size 0.8) (drill 0.4) (layers "F.Cu" "B.Cu") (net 2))
 (via (at 151.5 107.9) (size 0.8) (drill 0.4) (layers "F.Cu" "B.Cu") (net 2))
 (via (at 153.06 104.25) (size 0.8) (drill 0.4) (layers "F.Cu" "B.Cu") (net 2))
 (via (at 153.659999 102.75) (size 0.8) (drill 0.4) (layers "F.Cu" "B.Cu") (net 2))
 (segment (start 155.585 103.525) (end 156.385 102.725) (width 0.3) (layer "F.Cu") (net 3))
 (segment (start 156.2 105.65) (end 155.585 105.035) (width 0.3) (layer "F.Cu") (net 3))
 (segment (start 155.86 105.99) (end 156.2 105.65) (width 0.3) (layer "F.Cu") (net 3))
 (segment (start 155.86 107.2125) (end 155.86 105.99) (width 0.3) (layer "F.Cu") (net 3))
 (segment (start 155.585 105.035) (end 155.585 103.525) (width 0.3) (layer "F.Cu") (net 3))
 (segment (start 154.535 104.175) (end 154.535 104.833528) (width 0.5) (layer "F.Cu") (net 1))
 (segment (start 154.535 104.833528) (end 155.105736 105.404264) (width 0.5) (layer "F.Cu") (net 1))
 (segment (start 155.36 107.2125) (end 155.36 105.87) (width 0.3) (layer "F.Cu") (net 1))
 (segment (start 155.36 105.87) (end 155.14 105.65) (width 0.3) (layer "F.Cu") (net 1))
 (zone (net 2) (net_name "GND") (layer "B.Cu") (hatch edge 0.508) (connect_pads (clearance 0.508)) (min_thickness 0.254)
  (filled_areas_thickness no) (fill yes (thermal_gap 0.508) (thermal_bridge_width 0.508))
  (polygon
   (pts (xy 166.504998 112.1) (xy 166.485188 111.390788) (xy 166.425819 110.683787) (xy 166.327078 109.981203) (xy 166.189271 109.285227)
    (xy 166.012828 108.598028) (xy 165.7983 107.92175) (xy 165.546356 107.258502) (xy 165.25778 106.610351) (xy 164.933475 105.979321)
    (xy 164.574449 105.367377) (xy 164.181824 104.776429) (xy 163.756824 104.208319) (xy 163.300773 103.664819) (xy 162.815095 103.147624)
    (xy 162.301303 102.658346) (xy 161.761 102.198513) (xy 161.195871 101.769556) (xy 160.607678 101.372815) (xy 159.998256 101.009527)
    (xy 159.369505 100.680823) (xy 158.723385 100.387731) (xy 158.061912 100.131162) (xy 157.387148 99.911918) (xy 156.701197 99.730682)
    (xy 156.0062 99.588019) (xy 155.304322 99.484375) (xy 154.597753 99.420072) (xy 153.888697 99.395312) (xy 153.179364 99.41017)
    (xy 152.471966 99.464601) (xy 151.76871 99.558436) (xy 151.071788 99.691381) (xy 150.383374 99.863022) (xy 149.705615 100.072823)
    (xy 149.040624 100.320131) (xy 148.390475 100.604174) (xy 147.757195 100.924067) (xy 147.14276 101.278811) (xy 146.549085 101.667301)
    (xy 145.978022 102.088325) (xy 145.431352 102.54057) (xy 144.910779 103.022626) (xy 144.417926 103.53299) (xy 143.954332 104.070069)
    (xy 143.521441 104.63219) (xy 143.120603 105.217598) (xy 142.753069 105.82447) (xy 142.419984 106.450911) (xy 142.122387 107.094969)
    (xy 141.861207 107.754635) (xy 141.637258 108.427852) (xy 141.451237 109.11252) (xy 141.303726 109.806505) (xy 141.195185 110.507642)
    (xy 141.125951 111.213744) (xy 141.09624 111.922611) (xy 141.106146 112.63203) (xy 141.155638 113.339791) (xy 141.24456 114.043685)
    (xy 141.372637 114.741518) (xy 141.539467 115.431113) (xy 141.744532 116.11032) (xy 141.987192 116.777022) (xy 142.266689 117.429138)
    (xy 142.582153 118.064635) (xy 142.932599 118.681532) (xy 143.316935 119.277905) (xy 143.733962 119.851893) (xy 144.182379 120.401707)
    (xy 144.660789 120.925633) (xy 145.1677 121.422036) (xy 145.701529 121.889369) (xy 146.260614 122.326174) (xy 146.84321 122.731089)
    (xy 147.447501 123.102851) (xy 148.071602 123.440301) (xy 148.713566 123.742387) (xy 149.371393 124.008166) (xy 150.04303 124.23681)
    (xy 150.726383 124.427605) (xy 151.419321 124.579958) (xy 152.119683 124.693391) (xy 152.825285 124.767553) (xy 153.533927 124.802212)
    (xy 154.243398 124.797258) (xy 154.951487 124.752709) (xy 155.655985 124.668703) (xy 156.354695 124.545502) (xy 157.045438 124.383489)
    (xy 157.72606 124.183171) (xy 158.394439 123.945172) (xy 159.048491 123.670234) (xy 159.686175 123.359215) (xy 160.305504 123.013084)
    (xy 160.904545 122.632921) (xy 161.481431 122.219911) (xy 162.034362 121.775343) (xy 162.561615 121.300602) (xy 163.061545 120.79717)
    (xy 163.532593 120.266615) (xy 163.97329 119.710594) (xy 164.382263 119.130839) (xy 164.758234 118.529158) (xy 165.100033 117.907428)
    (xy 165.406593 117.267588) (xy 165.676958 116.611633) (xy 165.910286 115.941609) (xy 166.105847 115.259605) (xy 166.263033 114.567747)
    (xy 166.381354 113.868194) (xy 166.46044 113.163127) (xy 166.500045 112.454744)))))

